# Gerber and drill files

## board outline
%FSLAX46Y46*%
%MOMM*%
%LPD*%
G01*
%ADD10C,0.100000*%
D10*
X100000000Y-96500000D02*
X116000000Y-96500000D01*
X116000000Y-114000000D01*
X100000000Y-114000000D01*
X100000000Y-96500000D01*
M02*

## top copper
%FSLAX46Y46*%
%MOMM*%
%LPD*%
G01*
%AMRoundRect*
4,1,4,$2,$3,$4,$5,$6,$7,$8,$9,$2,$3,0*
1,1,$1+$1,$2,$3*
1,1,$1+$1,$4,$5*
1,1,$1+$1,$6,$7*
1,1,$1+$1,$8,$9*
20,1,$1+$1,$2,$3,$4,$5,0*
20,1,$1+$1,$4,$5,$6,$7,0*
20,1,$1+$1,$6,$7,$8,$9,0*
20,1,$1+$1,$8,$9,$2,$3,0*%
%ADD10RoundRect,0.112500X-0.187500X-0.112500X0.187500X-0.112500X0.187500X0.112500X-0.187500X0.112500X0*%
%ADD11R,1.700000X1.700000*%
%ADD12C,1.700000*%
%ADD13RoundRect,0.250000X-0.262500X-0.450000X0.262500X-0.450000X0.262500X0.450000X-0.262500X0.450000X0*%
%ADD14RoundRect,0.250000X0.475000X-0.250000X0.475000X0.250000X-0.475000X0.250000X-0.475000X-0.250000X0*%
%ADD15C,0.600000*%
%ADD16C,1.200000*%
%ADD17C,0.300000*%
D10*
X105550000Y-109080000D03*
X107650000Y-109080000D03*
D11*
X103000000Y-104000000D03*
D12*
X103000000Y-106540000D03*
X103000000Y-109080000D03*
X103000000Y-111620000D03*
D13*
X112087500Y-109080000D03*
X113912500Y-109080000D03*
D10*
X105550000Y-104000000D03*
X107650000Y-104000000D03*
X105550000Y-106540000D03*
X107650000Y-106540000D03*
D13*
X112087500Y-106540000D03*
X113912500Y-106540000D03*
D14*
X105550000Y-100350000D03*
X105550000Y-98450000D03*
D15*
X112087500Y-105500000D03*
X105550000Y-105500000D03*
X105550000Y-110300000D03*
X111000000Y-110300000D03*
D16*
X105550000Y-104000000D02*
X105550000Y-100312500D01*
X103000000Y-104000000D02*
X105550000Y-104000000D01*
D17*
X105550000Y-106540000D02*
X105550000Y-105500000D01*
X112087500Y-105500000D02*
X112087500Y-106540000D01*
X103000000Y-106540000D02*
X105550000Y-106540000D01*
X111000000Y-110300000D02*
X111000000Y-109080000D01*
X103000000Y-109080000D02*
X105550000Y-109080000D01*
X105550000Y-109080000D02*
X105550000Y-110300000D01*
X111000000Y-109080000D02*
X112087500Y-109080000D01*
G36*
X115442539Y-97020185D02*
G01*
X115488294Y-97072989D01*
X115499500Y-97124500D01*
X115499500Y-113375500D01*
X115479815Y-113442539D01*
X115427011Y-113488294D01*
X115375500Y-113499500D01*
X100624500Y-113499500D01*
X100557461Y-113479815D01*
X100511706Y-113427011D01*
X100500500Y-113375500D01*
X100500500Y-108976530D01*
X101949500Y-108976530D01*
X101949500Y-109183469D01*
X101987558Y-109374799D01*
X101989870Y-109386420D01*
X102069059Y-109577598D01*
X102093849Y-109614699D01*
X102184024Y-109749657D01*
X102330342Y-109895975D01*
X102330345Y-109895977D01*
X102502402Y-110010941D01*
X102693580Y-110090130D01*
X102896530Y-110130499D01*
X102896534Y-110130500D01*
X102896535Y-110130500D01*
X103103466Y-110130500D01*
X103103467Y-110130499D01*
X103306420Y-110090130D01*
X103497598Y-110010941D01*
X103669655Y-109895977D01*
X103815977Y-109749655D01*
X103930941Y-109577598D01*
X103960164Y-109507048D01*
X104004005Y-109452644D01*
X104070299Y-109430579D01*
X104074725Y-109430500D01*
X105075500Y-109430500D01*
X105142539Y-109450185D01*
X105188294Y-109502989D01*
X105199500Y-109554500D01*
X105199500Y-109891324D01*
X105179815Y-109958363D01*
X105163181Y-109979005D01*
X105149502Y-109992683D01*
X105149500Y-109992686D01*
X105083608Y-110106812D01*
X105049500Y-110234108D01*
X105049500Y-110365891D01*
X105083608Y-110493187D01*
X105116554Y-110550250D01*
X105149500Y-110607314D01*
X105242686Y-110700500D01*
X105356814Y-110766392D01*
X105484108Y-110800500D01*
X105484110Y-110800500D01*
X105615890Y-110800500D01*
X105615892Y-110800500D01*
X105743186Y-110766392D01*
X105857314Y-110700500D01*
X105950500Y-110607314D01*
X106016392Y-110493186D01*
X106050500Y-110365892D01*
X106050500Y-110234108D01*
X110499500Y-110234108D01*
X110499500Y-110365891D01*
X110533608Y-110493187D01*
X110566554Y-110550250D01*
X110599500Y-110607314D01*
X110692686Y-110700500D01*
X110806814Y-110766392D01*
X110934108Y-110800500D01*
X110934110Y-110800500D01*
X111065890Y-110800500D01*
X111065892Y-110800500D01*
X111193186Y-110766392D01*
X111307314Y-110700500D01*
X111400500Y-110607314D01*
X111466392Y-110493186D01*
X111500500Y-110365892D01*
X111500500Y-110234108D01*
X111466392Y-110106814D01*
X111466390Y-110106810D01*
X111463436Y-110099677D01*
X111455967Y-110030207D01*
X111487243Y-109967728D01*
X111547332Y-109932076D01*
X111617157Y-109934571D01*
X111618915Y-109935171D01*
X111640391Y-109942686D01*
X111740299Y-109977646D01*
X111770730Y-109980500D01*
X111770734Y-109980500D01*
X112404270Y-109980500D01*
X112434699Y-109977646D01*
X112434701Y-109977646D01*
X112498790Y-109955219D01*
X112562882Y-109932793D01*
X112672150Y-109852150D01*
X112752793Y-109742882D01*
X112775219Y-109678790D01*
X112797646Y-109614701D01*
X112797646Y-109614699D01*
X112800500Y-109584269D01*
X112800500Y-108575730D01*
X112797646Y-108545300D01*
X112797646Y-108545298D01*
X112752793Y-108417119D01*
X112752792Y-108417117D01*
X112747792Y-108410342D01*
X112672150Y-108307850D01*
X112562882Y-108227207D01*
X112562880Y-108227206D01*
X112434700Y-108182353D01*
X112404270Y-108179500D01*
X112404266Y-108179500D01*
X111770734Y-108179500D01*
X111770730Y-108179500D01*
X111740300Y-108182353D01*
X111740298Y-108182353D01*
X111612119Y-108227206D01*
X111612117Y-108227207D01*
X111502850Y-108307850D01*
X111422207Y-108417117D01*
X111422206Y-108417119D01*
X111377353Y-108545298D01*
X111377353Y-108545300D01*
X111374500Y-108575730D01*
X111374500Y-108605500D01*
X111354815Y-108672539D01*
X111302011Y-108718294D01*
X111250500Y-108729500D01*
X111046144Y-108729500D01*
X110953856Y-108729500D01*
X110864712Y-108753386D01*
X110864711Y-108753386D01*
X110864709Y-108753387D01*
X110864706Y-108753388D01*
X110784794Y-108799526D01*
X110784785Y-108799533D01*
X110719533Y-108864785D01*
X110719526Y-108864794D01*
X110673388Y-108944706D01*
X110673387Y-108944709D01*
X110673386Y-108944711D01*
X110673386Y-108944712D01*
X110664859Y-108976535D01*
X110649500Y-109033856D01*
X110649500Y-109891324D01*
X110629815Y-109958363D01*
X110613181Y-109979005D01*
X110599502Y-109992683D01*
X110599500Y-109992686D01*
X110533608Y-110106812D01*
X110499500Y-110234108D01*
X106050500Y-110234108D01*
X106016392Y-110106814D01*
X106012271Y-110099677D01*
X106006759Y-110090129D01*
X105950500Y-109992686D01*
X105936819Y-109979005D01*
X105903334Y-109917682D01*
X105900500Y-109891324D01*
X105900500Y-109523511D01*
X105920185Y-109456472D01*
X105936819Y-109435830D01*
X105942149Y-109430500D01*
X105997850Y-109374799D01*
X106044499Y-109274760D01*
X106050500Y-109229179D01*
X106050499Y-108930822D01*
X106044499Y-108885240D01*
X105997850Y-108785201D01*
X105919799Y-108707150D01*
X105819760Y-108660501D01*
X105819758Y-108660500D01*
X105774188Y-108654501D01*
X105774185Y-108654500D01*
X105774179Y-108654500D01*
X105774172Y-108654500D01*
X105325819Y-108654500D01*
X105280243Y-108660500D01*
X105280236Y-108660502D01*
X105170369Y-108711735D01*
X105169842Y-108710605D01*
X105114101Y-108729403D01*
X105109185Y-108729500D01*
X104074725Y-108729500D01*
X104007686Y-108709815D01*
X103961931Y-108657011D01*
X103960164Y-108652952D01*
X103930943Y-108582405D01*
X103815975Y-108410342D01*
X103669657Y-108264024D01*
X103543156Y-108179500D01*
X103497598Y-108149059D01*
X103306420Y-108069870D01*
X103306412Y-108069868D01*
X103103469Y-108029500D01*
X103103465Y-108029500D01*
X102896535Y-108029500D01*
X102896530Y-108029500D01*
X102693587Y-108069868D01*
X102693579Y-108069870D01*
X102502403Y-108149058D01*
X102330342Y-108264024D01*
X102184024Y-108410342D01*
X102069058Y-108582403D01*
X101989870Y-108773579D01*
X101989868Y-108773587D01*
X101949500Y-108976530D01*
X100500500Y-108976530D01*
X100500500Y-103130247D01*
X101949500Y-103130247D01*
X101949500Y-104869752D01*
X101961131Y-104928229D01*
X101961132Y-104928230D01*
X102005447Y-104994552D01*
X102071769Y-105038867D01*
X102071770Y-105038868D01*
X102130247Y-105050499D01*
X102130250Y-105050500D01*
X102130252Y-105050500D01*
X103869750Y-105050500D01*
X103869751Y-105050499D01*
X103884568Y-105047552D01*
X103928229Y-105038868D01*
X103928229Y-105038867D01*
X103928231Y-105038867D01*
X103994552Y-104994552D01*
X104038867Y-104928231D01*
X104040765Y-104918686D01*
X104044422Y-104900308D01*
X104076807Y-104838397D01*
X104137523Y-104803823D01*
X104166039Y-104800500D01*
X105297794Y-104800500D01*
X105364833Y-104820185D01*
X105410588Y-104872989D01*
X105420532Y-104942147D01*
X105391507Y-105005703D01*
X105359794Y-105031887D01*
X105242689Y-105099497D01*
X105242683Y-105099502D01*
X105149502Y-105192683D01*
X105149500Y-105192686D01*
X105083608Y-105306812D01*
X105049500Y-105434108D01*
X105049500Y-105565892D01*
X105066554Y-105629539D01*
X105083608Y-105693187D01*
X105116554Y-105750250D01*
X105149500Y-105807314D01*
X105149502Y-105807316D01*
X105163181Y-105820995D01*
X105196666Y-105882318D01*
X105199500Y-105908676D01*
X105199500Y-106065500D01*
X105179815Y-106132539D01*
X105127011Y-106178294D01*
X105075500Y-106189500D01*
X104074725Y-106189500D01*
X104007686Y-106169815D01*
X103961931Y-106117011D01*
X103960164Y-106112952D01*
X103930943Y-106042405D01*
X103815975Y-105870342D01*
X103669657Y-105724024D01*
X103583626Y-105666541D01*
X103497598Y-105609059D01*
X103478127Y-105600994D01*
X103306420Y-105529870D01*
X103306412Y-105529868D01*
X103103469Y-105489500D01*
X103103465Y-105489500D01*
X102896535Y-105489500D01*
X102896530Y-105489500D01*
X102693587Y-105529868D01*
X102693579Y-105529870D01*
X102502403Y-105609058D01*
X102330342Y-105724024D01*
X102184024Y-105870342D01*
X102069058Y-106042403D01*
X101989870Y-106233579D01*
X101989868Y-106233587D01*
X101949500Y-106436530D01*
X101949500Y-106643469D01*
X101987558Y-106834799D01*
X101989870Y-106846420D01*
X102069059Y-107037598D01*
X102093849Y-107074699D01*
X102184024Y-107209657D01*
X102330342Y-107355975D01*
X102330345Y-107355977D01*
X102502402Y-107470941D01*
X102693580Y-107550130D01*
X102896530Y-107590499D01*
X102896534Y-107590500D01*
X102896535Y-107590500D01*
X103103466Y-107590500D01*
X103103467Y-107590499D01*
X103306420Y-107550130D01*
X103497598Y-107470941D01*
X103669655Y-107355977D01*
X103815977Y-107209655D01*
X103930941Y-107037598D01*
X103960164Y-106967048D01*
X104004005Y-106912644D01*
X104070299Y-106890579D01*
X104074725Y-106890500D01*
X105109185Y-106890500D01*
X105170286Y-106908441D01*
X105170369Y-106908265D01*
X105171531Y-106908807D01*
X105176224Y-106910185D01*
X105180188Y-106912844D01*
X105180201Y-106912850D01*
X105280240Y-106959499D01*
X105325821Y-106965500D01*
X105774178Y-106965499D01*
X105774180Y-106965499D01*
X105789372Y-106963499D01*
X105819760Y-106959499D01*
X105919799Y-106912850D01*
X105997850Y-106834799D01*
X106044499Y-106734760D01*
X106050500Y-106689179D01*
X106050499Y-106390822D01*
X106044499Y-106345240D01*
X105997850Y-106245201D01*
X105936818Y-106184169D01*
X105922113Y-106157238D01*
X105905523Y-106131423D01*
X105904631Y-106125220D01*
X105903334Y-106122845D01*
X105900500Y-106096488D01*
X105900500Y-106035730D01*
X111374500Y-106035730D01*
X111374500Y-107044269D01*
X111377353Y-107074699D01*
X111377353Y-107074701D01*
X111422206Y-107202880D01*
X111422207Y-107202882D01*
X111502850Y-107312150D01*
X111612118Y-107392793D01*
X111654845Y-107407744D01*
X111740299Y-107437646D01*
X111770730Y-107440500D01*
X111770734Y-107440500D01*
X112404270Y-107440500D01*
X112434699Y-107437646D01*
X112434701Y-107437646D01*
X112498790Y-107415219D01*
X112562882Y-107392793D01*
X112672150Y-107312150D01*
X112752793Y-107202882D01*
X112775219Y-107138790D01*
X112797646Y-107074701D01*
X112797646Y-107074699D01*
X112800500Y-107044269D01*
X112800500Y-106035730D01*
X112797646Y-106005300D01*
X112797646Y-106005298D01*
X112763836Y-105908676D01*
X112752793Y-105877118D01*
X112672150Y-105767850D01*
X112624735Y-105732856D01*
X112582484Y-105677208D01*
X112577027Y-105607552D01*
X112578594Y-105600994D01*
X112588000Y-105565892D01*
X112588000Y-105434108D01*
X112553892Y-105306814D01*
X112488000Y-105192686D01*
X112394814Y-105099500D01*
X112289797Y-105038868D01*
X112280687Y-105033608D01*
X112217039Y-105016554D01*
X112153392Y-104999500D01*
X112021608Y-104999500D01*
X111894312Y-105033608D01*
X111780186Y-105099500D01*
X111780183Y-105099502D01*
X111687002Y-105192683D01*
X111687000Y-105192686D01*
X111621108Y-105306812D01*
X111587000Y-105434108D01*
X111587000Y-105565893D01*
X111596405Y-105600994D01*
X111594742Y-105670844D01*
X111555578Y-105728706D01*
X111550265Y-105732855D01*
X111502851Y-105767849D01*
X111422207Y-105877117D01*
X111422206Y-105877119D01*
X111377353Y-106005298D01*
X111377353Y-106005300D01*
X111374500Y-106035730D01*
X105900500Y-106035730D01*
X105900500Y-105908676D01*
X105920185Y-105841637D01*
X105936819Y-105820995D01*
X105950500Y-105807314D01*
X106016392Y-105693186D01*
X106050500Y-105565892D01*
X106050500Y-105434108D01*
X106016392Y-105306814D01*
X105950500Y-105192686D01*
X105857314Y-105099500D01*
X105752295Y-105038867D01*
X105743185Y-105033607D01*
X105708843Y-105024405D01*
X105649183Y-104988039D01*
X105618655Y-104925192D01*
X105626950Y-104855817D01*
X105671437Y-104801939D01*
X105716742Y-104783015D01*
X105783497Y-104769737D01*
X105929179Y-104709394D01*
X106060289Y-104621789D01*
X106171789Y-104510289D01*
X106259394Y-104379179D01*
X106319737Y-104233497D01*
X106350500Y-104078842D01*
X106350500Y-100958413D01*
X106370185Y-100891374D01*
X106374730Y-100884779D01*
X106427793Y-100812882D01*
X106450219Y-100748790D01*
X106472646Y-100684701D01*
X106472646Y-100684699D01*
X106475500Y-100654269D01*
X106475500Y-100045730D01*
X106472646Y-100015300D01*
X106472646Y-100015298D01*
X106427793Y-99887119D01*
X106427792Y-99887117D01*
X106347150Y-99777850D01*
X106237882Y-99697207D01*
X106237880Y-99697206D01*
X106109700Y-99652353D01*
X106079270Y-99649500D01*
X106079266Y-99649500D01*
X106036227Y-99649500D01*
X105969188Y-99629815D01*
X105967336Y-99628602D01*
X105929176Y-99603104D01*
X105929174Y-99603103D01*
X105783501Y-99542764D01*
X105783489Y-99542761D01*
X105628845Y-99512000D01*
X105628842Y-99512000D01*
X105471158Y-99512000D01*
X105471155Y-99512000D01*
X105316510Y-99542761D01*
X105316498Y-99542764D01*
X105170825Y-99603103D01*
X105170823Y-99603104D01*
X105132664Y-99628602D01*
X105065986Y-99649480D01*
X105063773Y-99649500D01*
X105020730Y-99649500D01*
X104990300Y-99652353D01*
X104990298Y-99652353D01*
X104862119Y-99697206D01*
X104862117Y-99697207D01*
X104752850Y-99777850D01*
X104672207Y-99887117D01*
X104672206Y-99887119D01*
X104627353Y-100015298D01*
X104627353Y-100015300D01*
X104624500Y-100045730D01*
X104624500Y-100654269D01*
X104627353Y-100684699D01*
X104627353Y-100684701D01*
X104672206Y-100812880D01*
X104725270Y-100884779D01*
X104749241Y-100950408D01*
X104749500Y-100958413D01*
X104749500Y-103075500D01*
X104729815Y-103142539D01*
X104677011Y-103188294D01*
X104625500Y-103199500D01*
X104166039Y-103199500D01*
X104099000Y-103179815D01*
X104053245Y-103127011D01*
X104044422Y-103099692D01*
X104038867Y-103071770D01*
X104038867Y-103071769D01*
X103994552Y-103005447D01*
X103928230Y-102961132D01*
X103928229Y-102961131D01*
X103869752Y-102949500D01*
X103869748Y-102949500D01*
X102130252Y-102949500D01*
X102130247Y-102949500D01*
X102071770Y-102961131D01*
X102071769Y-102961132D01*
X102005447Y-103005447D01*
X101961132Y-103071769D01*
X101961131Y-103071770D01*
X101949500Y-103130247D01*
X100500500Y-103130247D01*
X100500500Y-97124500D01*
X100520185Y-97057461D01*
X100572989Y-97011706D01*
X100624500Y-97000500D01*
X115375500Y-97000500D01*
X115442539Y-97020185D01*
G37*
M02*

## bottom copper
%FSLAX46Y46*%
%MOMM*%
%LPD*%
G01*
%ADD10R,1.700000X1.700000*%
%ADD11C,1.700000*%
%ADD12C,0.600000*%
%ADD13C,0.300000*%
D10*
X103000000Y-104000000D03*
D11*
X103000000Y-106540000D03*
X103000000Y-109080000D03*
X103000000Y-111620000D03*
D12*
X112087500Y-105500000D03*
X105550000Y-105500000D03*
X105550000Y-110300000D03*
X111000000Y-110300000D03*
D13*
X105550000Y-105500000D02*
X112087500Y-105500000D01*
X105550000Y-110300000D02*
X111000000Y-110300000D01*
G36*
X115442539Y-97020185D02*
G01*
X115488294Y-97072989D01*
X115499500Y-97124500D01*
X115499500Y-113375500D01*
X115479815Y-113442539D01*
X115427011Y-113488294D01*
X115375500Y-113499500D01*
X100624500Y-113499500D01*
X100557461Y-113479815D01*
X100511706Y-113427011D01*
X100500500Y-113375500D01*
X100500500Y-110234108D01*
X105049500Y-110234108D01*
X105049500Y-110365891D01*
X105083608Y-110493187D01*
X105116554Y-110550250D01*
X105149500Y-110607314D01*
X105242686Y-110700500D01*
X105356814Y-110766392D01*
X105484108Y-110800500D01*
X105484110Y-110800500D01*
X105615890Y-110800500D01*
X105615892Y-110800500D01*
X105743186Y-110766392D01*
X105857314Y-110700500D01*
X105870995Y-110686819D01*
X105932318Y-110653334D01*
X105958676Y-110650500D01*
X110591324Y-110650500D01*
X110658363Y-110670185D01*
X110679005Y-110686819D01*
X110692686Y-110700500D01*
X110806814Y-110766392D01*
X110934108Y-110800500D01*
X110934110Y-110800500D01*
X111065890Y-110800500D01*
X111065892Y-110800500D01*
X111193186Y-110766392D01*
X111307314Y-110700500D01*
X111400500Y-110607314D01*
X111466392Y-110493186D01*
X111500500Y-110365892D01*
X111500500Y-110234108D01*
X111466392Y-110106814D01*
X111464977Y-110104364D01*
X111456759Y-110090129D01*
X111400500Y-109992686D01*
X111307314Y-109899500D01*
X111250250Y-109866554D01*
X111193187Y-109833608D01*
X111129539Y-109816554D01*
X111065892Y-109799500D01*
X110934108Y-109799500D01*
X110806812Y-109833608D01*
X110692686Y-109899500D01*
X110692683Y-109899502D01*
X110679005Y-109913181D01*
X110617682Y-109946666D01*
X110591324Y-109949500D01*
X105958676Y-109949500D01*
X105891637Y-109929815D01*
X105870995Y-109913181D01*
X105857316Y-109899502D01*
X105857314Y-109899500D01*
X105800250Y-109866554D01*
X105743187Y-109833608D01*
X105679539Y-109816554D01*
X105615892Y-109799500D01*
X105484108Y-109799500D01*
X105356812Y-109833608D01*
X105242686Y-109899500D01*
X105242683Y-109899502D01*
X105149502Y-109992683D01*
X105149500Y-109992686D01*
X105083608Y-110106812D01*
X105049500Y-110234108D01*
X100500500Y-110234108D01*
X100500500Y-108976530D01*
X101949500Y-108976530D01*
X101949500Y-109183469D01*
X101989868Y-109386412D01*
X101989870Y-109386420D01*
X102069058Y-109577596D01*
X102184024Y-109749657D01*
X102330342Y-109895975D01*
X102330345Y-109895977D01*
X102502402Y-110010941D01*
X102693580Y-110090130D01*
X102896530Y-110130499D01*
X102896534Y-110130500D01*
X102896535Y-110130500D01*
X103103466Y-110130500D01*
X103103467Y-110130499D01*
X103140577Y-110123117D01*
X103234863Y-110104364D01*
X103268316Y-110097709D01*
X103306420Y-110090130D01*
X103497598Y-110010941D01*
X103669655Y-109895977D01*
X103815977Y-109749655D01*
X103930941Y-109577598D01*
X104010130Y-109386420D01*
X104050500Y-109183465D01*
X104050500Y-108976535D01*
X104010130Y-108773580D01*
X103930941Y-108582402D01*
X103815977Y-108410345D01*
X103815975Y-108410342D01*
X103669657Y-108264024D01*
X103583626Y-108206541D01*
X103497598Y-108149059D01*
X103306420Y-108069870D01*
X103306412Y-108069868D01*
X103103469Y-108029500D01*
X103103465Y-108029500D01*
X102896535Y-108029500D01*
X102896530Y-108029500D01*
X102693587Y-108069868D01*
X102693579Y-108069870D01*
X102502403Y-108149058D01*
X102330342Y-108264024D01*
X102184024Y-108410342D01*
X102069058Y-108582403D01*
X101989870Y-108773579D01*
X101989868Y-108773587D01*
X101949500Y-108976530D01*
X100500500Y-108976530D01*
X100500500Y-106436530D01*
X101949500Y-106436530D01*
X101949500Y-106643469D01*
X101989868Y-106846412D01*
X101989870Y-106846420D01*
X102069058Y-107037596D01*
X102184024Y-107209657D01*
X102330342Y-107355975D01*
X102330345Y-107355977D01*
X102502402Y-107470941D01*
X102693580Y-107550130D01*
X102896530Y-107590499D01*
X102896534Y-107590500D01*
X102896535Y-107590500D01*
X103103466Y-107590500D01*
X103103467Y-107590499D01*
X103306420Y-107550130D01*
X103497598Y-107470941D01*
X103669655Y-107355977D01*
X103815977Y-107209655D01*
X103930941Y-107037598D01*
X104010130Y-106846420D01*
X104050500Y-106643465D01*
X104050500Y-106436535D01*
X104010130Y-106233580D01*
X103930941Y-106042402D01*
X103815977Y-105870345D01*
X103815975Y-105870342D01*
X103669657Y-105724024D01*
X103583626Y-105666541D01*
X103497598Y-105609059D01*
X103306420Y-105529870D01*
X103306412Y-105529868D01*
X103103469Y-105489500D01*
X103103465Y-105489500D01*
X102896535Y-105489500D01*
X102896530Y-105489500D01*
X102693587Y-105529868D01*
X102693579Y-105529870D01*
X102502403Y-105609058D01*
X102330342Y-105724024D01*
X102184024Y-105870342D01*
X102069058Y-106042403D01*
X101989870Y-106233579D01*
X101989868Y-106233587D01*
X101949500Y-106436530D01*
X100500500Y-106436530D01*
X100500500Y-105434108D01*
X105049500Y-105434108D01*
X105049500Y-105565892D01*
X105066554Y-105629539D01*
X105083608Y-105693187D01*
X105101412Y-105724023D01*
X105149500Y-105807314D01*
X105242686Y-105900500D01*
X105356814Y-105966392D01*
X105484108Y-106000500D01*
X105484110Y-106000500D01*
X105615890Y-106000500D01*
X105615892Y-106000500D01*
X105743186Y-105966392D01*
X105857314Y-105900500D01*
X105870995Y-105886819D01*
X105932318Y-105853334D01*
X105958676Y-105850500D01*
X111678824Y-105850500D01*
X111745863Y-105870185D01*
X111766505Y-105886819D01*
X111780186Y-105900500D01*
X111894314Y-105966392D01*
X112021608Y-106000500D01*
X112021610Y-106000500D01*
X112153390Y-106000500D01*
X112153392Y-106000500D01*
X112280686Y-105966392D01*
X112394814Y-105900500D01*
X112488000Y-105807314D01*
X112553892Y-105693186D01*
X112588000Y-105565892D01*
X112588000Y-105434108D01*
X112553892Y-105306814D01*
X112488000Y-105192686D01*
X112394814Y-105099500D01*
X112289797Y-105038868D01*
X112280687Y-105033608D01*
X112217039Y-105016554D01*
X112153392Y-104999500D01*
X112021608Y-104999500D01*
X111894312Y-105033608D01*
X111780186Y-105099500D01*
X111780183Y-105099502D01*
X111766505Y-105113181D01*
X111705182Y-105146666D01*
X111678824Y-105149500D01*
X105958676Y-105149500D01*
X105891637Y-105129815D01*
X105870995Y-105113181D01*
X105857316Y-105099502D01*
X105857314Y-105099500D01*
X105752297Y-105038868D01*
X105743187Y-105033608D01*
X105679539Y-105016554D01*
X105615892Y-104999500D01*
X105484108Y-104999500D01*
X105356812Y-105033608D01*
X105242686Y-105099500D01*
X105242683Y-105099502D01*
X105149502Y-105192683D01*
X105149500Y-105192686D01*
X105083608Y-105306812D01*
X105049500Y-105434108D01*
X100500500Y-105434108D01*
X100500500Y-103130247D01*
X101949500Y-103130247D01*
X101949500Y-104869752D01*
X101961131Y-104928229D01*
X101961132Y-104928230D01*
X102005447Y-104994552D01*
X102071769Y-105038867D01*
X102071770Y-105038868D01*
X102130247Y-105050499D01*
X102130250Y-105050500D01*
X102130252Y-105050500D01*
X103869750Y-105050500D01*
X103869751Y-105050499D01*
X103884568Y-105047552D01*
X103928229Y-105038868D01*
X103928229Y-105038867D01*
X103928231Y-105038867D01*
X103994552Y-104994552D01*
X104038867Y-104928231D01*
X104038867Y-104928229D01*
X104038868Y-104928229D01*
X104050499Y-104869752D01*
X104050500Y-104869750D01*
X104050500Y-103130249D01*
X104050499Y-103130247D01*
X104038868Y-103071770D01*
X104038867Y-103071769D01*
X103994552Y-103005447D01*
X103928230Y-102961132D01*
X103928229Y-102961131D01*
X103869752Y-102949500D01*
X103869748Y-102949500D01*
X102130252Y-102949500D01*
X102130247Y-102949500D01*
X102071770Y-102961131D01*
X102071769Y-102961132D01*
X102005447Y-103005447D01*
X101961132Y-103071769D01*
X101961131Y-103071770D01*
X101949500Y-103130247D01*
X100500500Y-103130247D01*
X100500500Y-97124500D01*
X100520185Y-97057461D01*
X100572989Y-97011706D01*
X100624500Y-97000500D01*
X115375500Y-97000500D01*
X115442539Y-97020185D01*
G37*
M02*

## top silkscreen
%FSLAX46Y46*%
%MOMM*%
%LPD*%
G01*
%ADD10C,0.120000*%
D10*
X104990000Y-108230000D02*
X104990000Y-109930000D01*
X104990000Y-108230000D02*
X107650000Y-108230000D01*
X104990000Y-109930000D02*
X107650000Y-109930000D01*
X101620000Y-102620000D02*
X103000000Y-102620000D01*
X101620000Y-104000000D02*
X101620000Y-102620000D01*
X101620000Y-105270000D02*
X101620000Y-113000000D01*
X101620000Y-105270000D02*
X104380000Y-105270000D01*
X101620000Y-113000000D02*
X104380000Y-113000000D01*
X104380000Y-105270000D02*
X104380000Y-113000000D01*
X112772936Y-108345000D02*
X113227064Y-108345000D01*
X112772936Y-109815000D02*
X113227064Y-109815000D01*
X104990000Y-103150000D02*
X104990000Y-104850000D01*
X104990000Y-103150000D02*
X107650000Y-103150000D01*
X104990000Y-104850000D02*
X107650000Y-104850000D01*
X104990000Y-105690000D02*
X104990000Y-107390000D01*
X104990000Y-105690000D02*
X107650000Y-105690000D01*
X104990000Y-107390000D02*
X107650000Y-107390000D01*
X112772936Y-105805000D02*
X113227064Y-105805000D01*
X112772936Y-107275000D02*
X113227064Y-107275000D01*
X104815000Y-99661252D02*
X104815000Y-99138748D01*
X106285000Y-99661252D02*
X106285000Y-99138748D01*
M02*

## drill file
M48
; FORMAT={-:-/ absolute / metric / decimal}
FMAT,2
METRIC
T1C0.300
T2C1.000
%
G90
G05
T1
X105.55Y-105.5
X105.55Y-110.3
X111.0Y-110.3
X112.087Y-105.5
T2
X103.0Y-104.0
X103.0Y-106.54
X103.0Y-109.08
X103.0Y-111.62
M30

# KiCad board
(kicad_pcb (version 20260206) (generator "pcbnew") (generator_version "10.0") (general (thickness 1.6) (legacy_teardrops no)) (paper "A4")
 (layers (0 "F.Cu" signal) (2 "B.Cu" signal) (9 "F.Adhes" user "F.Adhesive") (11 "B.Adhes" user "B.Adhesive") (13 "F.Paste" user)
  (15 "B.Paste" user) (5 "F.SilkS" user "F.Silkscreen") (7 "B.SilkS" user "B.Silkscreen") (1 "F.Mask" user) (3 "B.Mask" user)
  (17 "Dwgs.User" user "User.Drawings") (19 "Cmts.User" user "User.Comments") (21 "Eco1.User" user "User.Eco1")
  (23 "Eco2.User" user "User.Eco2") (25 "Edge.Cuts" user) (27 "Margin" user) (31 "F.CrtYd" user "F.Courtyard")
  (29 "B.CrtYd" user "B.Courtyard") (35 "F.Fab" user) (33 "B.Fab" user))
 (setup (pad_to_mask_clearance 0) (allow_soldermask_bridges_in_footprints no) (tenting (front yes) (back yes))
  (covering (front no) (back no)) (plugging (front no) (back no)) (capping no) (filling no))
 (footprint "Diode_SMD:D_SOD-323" (layer "F.Cu") (at 106.6 109.08)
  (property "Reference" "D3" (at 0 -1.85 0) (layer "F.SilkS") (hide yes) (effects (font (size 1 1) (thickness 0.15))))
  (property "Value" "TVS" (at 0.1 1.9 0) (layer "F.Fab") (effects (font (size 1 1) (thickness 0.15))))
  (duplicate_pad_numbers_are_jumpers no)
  (fp_line (start -1.61 -0.85) (end -1.61 0.85) (stroke (width 0.12) (type solid)) (layer "F.SilkS"))
  (fp_line (start -1.61 -0.85) (end 1.05 -0.85) (stroke (width 0.12) (type solid)) (layer "F.SilkS"))
  (fp_line (start -1.61 0.85) (end 1.05 0.85) (stroke (width 0.12) (type solid)) (layer "F.SilkS"))
  (pad "1" smd roundrect (at -1.05 0) (size 0.6 0.45) (layers "F.Cu" "F.Mask" "F.Paste") (roundrect_rratio 0.25) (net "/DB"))
  (pad "2" smd roundrect (at 1.05 0) (size 0.6 0.45) (layers "F.Cu" "F.Mask" "F.Paste") (roundrect_rratio 0.25) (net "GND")))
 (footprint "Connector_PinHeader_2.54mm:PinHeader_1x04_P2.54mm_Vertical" (layer "F.Cu") (at 103 104)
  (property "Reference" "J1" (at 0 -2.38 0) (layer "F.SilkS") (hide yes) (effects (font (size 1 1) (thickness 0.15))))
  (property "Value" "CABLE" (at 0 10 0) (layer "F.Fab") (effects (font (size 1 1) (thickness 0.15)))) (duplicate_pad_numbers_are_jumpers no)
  (fp_line (start -1.38 -1.38) (end 0 -1.38) (stroke (width 0.12) (type solid)) (layer "F.SilkS"))
  (fp_line (start -1.38 0) (end -1.38 -1.38) (stroke (width 0.12) (type solid)) (layer "F.SilkS"))
  (fp_line (start -1.38 1.27) (end -1.38 9) (stroke (width 0.12) (type solid)) (layer "F.SilkS"))
  (fp_line (start -1.38 1.27) (end 1.38 1.27) (stroke (width 0.12) (type solid)) (layer "F.SilkS"))
  (fp_line (start -1.38 9) (end 1.38 9) (stroke (width 0.12) (type solid)) (layer "F.SilkS"))
  (fp_line (start 1.38 1.27) (end 1.38 9) (stroke (width 0.12) (type solid)) (layer "F.SilkS"))
  (pad "1" thru_hole rect (at 0 0) (size 1.7 1.7) (drill 1) (layers "*.Cu" "*.Mask") (remove_unused_layers no) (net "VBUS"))
  (pad "2" thru_hole circle (at 0 2.54) (size 1.7 1.7) (drill 1) (layers "*.Cu" "*.Mask") (remove_unused_layers no) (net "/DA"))
  (pad "3" thru_hole circle (at 0 5.08) (size 1.7 1.7) (drill 1) (layers "*.Cu" "*.Mask") (remove_unused_layers no) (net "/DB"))
  (pad "4" thru_hole circle (at 0 7.62) (size 1.7 1.7) (drill 1) (layers "*.Cu" "*.Mask") (remove_unused_layers no) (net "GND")))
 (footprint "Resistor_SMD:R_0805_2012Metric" (layer "F.Cu") (at 113 109.08)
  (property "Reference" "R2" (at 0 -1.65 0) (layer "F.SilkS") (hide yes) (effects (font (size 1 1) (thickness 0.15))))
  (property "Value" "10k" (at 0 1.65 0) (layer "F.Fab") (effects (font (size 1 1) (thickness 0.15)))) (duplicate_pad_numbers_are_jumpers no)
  (fp_line (start -0.227064 -0.735) (end 0.227064 -0.735) (stroke (width 0.12) (type solid)) (layer "F.SilkS"))
  (fp_line (start -0.227064 0.735) (end 0.227064 0.735) (stroke (width 0.12) (type solid)) (layer "F.SilkS"))
  (pad "1" smd roundrect (at -0.9125 0) (size 1.025 1.4) (layers "F.Cu" "F.Mask" "F.Paste") (roundrect_rratio 0.243902) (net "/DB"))
  (pad "2" smd roundrect (at 0.9125 0) (size 1.025 1.4) (layers "F.Cu" "F.Mask" "F.Paste") (roundrect_rratio 0.243902) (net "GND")))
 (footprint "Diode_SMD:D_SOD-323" (layer "F.Cu") (at 106.6 104)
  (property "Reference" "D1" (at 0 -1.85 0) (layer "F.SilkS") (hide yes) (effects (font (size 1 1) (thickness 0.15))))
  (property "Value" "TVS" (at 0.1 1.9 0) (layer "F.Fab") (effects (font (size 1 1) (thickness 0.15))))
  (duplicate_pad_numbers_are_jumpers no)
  (fp_line (start -1.61 -0.85) (end -1.61 0.85) (stroke (width 0.12) (type solid)) (layer "F.SilkS"))
  (fp_line (start -1.61 -0.85) (end 1.05 -0.85) (stroke (width 0.12) (type solid)) (layer "F.SilkS"))
  (fp_line (start -1.61 0.85) (end 1.05 0.85) (stroke (width 0.12) (type solid)) (layer "F.SilkS"))
  (pad "1" smd roundrect (at -1.05 0) (size 0.6 0.45) (layers "F.Cu" "F.Mask" "F.Paste") (roundrect_rratio 0.25) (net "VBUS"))
  (pad "2" smd roundrect (at 1.05 0) (size 0.6 0.45) (layers "F.Cu" "F.Mask" "F.Paste") (roundrect_rratio 0.25) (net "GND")))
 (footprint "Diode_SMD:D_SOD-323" (layer "F.Cu") (at 106.6 106.54)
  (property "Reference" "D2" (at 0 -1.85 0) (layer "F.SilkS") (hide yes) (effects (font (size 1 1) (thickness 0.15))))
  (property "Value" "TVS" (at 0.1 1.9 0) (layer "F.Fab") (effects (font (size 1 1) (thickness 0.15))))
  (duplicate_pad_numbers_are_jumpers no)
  (fp_line (start -1.61 -0.85) (end -1.61 0.85) (stroke (width 0.12) (type solid)) (layer "F.SilkS"))
  (fp_line (start -1.61 -0.85) (end 1.05 -0.85) (stroke (width 0.12) (type solid)) (layer "F.SilkS"))
  (fp_line (start -1.61 0.85) (end 1.05 0.85) (stroke (width 0.12) (type solid)) (layer "F.SilkS"))
  (pad "1" smd roundrect (at -1.05 0) (size 0.6 0.45) (layers "F.Cu" "F.Mask" "F.Paste") (roundrect_rratio 0.25) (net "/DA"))
  (pad "2" smd roundrect (at 1.05 0) (size 0.6 0.45) (layers "F.Cu" "F.Mask" "F.Paste") (roundrect_rratio 0.25) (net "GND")))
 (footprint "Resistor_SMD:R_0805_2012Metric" (layer "F.Cu") (at 113 106.54)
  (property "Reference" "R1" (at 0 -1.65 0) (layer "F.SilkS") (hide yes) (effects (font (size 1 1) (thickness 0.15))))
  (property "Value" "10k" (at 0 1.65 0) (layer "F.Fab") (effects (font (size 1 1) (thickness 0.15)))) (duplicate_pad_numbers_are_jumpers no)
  (fp_line (start -0.227064 -0.735) (end 0.227064 -0.735) (stroke (width 0.12) (type solid)) (layer "F.SilkS"))
  (fp_line (start -0.227064 0.735) (end 0.227064 0.735) (stroke (width 0.12) (type solid)) (layer "F.SilkS"))
  (pad "1" smd roundrect (at -0.9125 0) (size 1.025 1.4) (layers "F.Cu" "F.Mask" "F.Paste") (roundrect_rratio 0.243902) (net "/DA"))
  (pad "2" smd roundrect (at 0.9125 0) (size 1.025 1.4) (layers "F.Cu" "F.Mask" "F.Paste") (roundrect_rratio 0.243902) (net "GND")))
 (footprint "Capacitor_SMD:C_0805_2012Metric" (layer "F.Cu") (at 105.55 99.4 90)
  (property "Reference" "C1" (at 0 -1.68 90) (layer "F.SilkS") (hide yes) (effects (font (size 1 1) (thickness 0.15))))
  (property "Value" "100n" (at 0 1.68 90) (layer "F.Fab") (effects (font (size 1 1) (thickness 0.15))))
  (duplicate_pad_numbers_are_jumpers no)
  (fp_line (start -0.261252 -0.735) (end 0.261252 -0.735) (stroke (width 0.12) (type solid)) (layer "F.SilkS"))
  (fp_line (start -0.261252 0.735) (end 0.261252 0.735) (stroke (width 0.12) (type solid)) (layer "F.SilkS"))
  (pad "1" smd roundrect (at -0.95 0 90) (size 1 1.45) (layers "F.Cu" "F.Mask" "F.Paste") (roundrect_rratio 0.25) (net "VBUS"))
  (pad "2" smd roundrect (at 0.95 0 90) (size 1 1.45) (layers "F.Cu" "F.Mask" "F.Paste") (roundrect_rratio 0.25) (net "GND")))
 (gr_rect (start 100 96.5) (end 116 114) (stroke (width 0.1) (type default)) (fill no) (layer "Edge.Cuts"))
 (segment (start 105.55 104) (end 105.55 100.3125) (width 1.2) (layer "F.Cu") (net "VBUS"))
 (segment (start 103 104) (end 105.55 104) (width 1.2) (layer "F.Cu") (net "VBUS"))
 (segment (start 105.55 106.54) (end 105.55 105.5) (width 0.3) (layer "F.Cu") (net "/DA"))
 (segment (start 112.0875 105.5) (end 112.0875 106.54) (width 0.3) (layer "F.Cu") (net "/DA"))
 (segment (start 103 106.54) (end 105.55 106.54) (width 0.3) (layer "F.Cu") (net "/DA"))
 (via (at 112.0875 105.5) (size 0.6) (drill 0.3) (layers "F.Cu" "B.Cu") (capping no) (covering (front no) (back no))
  (plugging (front no) (back no)) (filling no) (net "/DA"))
 (via (at 105.55 105.5) (size 0.6) (drill 0.3) (layers "F.Cu" "B.Cu") (capping no) (covering (front no) (back no))
  (plugging (front no) (back no)) (filling no) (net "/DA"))
 (segment (start 105.55 105.5) (end 112.0875 105.5) (width 0.3) (layer "B.Cu") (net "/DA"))
 (segment (start 111 110.3) (end 111 109.08) (width 0.3) (layer "F.Cu") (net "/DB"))
 (segment (start 103 109.08) (end 105.55 109.08) (width 0.3) (layer "F.Cu") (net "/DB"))
 (segment (start 105.55 109.08) (end 105.55 110.3) (width 0.3) (layer "F.Cu") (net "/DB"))
 (segment (start 111 109.08) (end 112.0875 109.08) (width 0.3) (layer "F.Cu") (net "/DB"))
 (via (at 105.55 110.3) (size 0.6) (drill 0.3) (layers "F.Cu" "B.Cu") (capping no) (covering (front no) (back no))
  (plugging (front no) (back no)) (filling no) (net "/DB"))
 (via (at 111 110.3) (size 0.6) (drill 0.3) (layers "F.Cu" "B.Cu") (capping no) (covering (front no) (back no))
  (plugging (front no) (back no)) (filling no) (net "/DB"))
 (segment (start 105.55 110.3) (end 111 110.3) (width 0.3) (layer "B.Cu") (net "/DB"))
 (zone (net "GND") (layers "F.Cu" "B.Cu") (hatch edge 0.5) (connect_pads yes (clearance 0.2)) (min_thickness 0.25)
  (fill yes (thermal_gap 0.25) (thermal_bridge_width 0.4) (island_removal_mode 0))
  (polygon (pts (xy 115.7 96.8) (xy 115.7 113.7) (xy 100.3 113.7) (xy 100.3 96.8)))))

